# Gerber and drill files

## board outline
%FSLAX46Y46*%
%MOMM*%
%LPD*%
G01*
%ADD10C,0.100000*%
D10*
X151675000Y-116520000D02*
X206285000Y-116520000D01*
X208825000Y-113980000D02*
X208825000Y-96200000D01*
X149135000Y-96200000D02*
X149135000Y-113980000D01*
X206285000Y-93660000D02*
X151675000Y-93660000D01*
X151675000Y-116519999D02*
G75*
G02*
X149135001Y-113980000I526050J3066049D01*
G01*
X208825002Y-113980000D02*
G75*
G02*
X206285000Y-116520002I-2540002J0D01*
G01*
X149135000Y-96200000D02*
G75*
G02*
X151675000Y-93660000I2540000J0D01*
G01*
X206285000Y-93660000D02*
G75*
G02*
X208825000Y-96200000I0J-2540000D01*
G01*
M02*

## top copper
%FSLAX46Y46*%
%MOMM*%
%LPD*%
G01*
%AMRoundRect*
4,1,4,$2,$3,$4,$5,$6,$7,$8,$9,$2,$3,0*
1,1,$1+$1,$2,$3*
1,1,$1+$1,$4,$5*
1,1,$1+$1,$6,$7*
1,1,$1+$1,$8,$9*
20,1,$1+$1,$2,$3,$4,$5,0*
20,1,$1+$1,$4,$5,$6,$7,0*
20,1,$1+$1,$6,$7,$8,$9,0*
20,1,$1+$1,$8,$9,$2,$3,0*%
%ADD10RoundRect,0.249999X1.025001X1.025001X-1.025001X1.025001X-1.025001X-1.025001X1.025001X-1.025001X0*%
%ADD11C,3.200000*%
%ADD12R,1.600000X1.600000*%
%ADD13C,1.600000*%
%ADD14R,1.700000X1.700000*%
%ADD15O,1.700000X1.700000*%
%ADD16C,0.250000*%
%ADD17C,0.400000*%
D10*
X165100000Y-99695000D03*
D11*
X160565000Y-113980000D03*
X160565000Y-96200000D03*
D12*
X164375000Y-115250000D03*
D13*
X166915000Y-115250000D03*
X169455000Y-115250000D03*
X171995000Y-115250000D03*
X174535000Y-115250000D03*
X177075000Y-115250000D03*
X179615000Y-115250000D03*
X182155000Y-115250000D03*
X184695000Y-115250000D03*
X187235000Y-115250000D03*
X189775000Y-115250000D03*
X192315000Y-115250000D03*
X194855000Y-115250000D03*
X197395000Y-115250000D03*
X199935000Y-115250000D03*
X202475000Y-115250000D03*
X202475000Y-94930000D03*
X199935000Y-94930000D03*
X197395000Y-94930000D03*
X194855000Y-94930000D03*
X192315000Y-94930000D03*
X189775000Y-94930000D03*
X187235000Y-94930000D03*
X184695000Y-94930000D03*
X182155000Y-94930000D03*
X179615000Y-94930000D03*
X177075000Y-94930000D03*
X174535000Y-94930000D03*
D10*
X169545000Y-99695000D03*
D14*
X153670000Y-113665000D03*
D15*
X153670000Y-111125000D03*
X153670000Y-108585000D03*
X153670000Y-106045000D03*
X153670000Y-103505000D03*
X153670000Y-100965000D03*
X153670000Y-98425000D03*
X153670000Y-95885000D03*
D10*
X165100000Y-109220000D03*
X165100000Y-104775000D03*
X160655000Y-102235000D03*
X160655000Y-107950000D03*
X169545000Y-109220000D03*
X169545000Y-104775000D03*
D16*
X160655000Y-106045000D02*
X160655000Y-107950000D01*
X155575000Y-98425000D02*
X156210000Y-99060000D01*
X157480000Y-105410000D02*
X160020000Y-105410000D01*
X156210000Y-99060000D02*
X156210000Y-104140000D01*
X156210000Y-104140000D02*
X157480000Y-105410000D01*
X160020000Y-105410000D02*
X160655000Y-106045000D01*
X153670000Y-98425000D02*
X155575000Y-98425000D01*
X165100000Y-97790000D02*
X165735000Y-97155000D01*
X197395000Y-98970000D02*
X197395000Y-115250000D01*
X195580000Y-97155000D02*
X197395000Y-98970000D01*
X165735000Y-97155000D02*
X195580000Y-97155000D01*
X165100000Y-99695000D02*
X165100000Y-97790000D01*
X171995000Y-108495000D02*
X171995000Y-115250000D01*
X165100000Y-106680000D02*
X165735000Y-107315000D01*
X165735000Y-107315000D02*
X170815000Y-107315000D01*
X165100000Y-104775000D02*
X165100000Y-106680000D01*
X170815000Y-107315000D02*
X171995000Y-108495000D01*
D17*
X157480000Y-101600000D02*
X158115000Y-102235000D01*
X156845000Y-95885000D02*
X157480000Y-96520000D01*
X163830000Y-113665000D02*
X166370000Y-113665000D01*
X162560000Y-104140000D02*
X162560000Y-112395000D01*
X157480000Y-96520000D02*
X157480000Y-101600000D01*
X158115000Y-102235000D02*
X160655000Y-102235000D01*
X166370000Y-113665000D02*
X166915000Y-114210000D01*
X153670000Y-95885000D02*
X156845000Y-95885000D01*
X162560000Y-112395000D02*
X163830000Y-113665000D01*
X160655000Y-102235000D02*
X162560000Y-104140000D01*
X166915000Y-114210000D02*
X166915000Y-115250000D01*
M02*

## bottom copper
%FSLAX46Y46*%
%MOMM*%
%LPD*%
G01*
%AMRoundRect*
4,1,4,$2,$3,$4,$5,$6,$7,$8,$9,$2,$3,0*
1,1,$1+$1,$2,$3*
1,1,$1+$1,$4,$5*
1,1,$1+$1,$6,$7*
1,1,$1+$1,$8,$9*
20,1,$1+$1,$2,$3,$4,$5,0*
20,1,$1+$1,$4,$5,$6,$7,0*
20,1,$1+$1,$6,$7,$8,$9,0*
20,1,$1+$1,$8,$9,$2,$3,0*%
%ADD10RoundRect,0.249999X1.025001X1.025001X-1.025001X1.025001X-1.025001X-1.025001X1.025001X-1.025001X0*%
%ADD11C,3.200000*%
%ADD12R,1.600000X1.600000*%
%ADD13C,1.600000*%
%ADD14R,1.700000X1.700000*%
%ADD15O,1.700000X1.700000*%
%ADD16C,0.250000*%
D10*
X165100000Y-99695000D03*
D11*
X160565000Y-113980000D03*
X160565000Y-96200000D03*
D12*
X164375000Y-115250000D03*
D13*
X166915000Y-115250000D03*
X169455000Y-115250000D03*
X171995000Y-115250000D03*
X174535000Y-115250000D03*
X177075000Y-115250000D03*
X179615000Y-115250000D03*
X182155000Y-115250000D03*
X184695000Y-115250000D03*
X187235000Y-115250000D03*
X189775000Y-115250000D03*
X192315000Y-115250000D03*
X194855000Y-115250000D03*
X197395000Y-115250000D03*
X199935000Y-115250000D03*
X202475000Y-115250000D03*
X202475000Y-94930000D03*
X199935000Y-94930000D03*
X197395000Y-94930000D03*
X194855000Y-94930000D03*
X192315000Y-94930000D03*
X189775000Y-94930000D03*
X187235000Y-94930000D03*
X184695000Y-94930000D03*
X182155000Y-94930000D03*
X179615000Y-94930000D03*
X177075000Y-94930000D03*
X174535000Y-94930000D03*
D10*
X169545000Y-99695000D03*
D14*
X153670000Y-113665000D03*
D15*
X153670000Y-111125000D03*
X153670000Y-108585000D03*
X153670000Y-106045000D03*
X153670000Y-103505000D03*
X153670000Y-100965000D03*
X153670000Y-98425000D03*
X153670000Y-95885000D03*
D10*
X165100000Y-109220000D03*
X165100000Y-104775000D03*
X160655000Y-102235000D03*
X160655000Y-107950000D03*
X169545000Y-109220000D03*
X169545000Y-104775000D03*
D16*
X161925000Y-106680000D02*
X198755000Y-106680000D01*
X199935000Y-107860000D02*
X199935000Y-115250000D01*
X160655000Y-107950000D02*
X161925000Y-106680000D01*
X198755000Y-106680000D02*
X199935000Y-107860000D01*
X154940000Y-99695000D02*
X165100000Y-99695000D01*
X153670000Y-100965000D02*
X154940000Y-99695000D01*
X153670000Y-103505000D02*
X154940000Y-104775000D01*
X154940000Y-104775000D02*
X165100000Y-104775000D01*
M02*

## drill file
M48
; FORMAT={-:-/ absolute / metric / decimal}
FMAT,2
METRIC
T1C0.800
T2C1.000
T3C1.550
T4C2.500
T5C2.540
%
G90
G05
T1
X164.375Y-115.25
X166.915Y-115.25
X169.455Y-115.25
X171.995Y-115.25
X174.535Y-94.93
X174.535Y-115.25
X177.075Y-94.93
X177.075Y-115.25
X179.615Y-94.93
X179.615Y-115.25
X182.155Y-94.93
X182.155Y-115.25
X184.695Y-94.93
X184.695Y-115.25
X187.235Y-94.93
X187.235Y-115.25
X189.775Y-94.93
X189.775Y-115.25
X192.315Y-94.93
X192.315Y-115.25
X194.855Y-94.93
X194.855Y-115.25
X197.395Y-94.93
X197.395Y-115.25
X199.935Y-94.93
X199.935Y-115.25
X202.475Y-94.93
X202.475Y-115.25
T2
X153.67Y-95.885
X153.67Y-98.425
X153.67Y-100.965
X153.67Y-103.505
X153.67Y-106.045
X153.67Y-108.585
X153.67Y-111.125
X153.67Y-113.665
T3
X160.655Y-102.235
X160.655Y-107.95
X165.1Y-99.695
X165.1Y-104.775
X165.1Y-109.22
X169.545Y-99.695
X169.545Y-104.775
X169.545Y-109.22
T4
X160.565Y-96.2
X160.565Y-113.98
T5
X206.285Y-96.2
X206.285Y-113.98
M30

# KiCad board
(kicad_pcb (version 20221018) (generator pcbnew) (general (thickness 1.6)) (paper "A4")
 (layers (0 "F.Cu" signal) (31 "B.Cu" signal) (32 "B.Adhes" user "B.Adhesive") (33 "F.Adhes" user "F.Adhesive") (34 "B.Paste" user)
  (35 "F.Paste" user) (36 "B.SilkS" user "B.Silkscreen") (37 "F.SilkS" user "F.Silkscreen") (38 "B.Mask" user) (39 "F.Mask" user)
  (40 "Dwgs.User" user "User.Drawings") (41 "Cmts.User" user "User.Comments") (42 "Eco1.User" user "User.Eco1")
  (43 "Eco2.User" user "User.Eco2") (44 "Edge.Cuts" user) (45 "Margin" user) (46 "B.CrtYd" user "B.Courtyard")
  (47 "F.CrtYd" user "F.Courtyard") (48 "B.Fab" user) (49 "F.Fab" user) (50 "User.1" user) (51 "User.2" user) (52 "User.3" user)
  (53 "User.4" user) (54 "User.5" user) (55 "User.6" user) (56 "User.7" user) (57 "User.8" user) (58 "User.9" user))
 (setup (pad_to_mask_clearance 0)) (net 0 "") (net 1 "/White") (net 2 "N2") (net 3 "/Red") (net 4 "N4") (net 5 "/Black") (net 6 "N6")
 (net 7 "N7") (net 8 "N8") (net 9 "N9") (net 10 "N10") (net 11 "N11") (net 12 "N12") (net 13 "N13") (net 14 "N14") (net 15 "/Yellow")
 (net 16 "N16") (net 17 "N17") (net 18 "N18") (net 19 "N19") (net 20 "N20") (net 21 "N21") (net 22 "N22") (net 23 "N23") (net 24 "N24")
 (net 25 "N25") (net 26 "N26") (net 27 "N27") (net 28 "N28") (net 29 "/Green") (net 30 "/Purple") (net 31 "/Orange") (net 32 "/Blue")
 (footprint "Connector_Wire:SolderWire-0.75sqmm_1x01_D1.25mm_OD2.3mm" (layer "F.Cu") (at 165.1 99.695 180)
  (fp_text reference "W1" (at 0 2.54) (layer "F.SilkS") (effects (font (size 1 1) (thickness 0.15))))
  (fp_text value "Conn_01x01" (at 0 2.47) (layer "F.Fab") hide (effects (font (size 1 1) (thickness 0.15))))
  (pad "1" thru_hole roundrect (at 0 0 180) (size 2.55 2.55) (drill 1.55) (layers "*.Cu" "*.Mask") (roundrect_rratio 0.098039)
   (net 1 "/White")))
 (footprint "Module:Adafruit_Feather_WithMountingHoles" (layer "F.Cu") (at 164.375 115.25 90)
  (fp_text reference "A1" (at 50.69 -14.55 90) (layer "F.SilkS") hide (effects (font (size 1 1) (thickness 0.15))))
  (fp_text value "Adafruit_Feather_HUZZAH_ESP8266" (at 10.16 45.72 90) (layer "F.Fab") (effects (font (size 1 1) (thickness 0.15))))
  (fp_line (start -1.27 -12.7) (end -1.27 41.91) (stroke (width 0.1) (type solid)) (layer "Edge.Cuts"))
  (fp_line (start 1.27 44.45) (end 19.05 44.45) (stroke (width 0.1) (type solid)) (layer "Edge.Cuts"))
  (fp_line (start 19.05 -15.24) (end 1.27 -15.24) (stroke (width 0.1) (type solid)) (layer "Edge.Cuts"))
  (fp_line (start 21.59 41.91) (end 21.59 -12.7) (stroke (width 0.1) (type solid)) (layer "Edge.Cuts"))
  (fp_arc (start -1.269999 -12.7) (mid -0.403653 -14.373653) (end 1.27 -15.239999) (stroke (width 0.1) (type solid)) (layer "Edge.Cuts"))
  (fp_arc (start 1.27 44.450002) (mid -0.526052 43.706052) (end -1.27 41.91) (stroke (width 0.1) (type solid)) (layer "Edge.Cuts"))
  (fp_arc (start 19.05 -15.24) (mid 20.846051 -14.496051) (end 21.59 -12.7) (stroke (width 0.1) (type solid)) (layer "Edge.Cuts"))
  (fp_arc (start 21.59 41.91) (mid 20.846051 43.706051) (end 19.05 44.45) (stroke (width 0.1) (type solid)) (layer "Edge.Cuts"))
  (pad "" np_thru_hole circle (at 1.27 -3.81) (size 3.2 3.2) (drill 2.5) (layers "*.Cu" "*.Mask"))
  (pad "" np_thru_hole circle (at 1.27 41.91) (size 2.54 2.54) (drill 2.54) (layers "*.Cu" "*.Mask"))
  (pad "" np_thru_hole circle (at 19.05 -3.81) (size 3.2 3.2) (drill 2.5) (layers "*.Cu" "*.Mask"))
  (pad "" np_thru_hole circle (at 19.05 41.91) (size 2.54 2.54) (drill 2.54) (layers "*.Cu" "*.Mask"))
  (pad "1" thru_hole rect (at 0 0 270) (size 1.6 1.6) (drill 0.8) (layers "*.Cu" "*.Mask") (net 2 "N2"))
  (pad "2" thru_hole circle (at 0 2.54 270) (size 1.6 1.6) (drill 0.8) (layers "*.Cu" "*.Mask") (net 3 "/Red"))
  (pad "3" thru_hole circle (at 0 5.08 270) (size 1.6 1.6) (drill 0.8) (layers "*.Cu" "*.Mask") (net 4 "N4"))
  (pad "4" thru_hole circle (at 0 7.62 270) (size 1.6 1.6) (drill 0.8) (layers "*.Cu" "*.Mask") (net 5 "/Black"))
  (pad "5" thru_hole circle (at 0 10.16 270) (size 1.6 1.6) (drill 0.8) (layers "*.Cu" "*.Mask") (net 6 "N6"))
  (pad "6" thru_hole circle (at 0 12.7 270) (size 1.6 1.6) (drill 0.8) (layers "*.Cu" "*.Mask") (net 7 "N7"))
  (pad "7" thru_hole circle (at 0 15.24 270) (size 1.6 1.6) (drill 0.8) (layers "*.Cu" "*.Mask") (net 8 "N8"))
  (pad "8" thru_hole circle (at 0 17.78 270) (size 1.6 1.6) (drill 0.8) (layers "*.Cu" "*.Mask") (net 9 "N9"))
  (pad "9" thru_hole circle (at 0 20.32 270) (size 1.6 1.6) (drill 0.8) (layers "*.Cu" "*.Mask") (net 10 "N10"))
  (pad "10" thru_hole circle (at 0 22.86 270) (size 1.6 1.6) (drill 0.8) (layers "*.Cu" "*.Mask") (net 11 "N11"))
  (pad "11" thru_hole circle (at 0 25.4 270) (size 1.6 1.6) (drill 0.8) (layers "*.Cu" "*.Mask") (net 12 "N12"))
  (pad "12" thru_hole circle (at 0 27.94 270) (size 1.6 1.6) (drill 0.8) (layers "*.Cu" "*.Mask") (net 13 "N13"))
  (pad "13" thru_hole circle (at 0 30.48 270) (size 1.6 1.6) (drill 0.8) (layers "*.Cu" "*.Mask") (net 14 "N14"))
  (pad "14" thru_hole circle (at 0 33.02 270) (size 1.6 1.6) (drill 0.8) (layers "*.Cu" "*.Mask") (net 1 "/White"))
  (pad "15" thru_hole circle (at 0 35.56 270) (size 1.6 1.6) (drill 0.8) (layers "*.Cu" "*.Mask") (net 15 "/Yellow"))
  (pad "16" thru_hole circle (at 0 38.1 270) (size 1.6 1.6) (drill 0.8) (layers "*.Cu" "*.Mask") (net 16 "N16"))
  (pad "17" thru_hole circle (at 20.32 38.1 270) (size 1.6 1.6) (drill 0.8) (layers "*.Cu" "*.Mask") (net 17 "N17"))
  (pad "18" thru_hole circle (at 20.32 35.56 270) (size 1.6 1.6) (drill 0.8) (layers "*.Cu" "*.Mask") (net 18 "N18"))
  (pad "19" thru_hole circle (at 20.32 33.02 270) (size 1.6 1.6) (drill 0.8) (layers "*.Cu" "*.Mask") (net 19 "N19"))
  (pad "20" thru_hole circle (at 20.32 30.48 270) (size 1.6 1.6) (drill 0.8) (layers "*.Cu" "*.Mask") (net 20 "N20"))
  (pad "21" thru_hole circle (at 20.32 27.94 270) (size 1.6 1.6) (drill 0.8) (layers "*.Cu" "*.Mask") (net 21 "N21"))
  (pad "22" thru_hole circle (at 20.32 25.4 270) (size 1.6 1.6) (drill 0.8) (layers "*.Cu" "*.Mask") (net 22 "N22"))
  (pad "23" thru_hole circle (at 20.32 22.86 270) (size 1.6 1.6) (drill 0.8) (layers "*.Cu" "*.Mask") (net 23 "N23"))
  (pad "24" thru_hole circle (at 20.32 20.32 270) (size 1.6 1.6) (drill 0.8) (layers "*.Cu" "*.Mask") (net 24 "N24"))
  (pad "25" thru_hole circle (at 20.32 17.78 270) (size 1.6 1.6) (drill 0.8) (layers "*.Cu" "*.Mask") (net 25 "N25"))
  (pad "26" thru_hole circle (at 20.32 15.24 270) (size 1.6 1.6) (drill 0.8) (layers "*.Cu" "*.Mask") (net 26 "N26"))
  (pad "27" thru_hole circle (at 20.32 12.7 270) (size 1.6 1.6) (drill 0.8) (layers "*.Cu" "*.Mask") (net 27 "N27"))
  (pad "28" thru_hole circle (at 20.32 10.16 270) (size 1.6 1.6) (drill 0.8) (layers "*.Cu" "*.Mask") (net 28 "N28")))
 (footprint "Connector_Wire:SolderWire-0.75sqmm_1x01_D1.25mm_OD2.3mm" (layer "F.Cu") (at 169.545 99.695 180)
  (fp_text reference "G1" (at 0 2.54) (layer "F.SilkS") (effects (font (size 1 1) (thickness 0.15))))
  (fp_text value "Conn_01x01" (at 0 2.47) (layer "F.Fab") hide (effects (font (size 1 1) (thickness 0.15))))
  (pad "1" thru_hole roundrect (at 0 0 180) (size 2.55 2.55) (drill 1.55) (layers "*.Cu" "*.Mask") (roundrect_rratio 0.098039)
   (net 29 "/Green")))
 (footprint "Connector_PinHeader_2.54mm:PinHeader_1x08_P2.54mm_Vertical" (layer "F.Cu") (at 153.67 113.665 180)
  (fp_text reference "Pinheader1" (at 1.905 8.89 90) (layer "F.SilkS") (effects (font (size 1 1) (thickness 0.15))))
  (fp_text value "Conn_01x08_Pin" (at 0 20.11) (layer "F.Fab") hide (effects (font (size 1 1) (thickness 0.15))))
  (pad "1" thru_hole rect (at 0 0 180) (size 1.7 1.7) (drill 1) (layers "*.Cu" "*.Mask") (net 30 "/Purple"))
  (pad "2" thru_hole oval (at 0 2.54 180) (size 1.7 1.7) (drill 1) (layers "*.Cu" "*.Mask") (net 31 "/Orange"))
  (pad "3" thru_hole oval (at 0 5.08 180) (size 1.7 1.7) (drill 1) (layers "*.Cu" "*.Mask") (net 29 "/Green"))
  (pad "4" thru_hole oval (at 0 7.62 180) (size 1.7 1.7) (drill 1) (layers "*.Cu" "*.Mask") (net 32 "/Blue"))
  (pad "5" thru_hole oval (at 0 10.16 180) (size 1.7 1.7) (drill 1) (layers "*.Cu" "*.Mask") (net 5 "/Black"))
  (pad "6" thru_hole oval (at 0 12.7 180) (size 1.7 1.7) (drill 1) (layers "*.Cu" "*.Mask") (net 1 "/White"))
  (pad "7" thru_hole oval (at 0 15.24 180) (size 1.7 1.7) (drill 1) (layers "*.Cu" "*.Mask") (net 15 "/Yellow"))
  (pad "8" thru_hole oval (at 0 17.78 180) (size 1.7 1.7) (drill 1) (layers "*.Cu" "*.Mask") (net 3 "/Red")))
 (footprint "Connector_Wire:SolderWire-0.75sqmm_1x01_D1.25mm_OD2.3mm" (layer "F.Cu") (at 165.1 109.22 180)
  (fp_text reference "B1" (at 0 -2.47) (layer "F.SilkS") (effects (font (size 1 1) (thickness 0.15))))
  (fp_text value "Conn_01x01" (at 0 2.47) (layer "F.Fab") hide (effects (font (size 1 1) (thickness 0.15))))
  (pad "1" thru_hole roundrect (at 0 0 180) (size 2.55 2.55) (drill 1.55) (layers "*.Cu" "*.Mask") (roundrect_rratio 0.098039)
   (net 32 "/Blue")))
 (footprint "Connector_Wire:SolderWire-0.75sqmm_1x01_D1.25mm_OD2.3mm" (layer "F.Cu") (at 165.1 104.775 180)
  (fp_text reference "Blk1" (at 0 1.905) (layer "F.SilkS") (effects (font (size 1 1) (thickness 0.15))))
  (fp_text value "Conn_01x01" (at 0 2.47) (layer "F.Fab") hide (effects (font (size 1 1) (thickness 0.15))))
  (pad "1" thru_hole roundrect (at 0 0 180) (size 2.55 2.55) (drill 1.55) (layers "*.Cu" "*.Mask") (roundrect_rratio 0.098039)
   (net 5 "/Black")))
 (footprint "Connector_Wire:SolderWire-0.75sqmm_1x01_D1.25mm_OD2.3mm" (layer "F.Cu") (at 160.655 102.235 180)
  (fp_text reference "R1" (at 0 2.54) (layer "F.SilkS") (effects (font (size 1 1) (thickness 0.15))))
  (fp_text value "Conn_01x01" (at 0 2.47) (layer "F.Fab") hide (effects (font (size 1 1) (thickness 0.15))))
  (pad "1" thru_hole roundrect (at 0 0 180) (size 2.55 2.55) (drill 1.55) (layers "*.Cu" "*.Mask") (roundrect_rratio 0.098039)
   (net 3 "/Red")))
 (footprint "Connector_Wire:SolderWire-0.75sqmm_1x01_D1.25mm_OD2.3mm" (layer "F.Cu") (at 160.655 107.95 180)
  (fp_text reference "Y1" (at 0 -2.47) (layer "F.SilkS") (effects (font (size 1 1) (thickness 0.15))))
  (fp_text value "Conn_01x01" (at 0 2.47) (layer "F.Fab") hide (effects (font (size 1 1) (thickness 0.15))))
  (pad "1" thru_hole roundrect (at 0 0 180) (size 2.55 2.55) (drill 1.55) (layers "*.Cu" "*.Mask") (roundrect_rratio 0.098039)
   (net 15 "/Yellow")))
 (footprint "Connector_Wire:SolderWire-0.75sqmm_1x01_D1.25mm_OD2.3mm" (layer "F.Cu") (at 169.545 109.22 180)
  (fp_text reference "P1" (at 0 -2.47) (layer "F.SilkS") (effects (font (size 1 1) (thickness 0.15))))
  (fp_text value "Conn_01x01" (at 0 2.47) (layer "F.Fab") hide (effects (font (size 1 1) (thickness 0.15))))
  (pad "1" thru_hole roundrect (at 0 0 180) (size 2.55 2.55) (drill 1.55) (layers "*.Cu" "*.Mask") (roundrect_rratio 0.098039)
   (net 30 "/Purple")))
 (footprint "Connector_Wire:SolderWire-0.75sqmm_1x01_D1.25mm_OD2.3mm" (layer "F.Cu") (at 169.545 104.775 180)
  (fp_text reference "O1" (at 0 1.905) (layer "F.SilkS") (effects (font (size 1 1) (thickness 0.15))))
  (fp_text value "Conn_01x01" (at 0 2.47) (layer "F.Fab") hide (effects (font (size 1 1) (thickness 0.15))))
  (pad "1" thru_hole roundrect (at 0 0 180) (size 2.55 2.55) (drill 1.55) (layers "*.Cu" "*.Mask") (roundrect_rratio 0.098039)
   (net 31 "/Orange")))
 (segment (start 160.655 106.045) (end 160.655 107.95) (width 0.25) (layer "F.Cu") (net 15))
 (segment (start 155.575 98.425) (end 156.21 99.06) (width 0.25) (layer "F.Cu") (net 15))
 (segment (start 157.48 105.41) (end 160.02 105.41) (width 0.25) (layer "F.Cu") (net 15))
 (segment (start 156.21 99.06) (end 156.21 104.14) (width 0.25) (layer "F.Cu") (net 15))
 (segment (start 156.21 104.14) (end 157.48 105.41) (width 0.25) (layer "F.Cu") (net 15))
 (segment (start 160.02 105.41) (end 160.655 106.045) (width 0.25) (layer "F.Cu") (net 15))
 (segment (start 153.67 98.425) (end 155.575 98.425) (width 0.25) (layer "F.Cu") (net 15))
 (segment (start 161.925 106.68) (end 198.755 106.68) (width 0.25) (layer "B.Cu") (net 15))
 (segment (start 199.935 107.86) (end 199.935 115.25) (width 0.25) (layer "B.Cu") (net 15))
 (segment (start 160.655 107.95) (end 161.925 106.68) (width 0.25) (layer "B.Cu") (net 15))
 (segment (start 198.755 106.68) (end 199.935 107.86) (width 0.25) (layer "B.Cu") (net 15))
 (segment (start 165.1 97.79) (end 165.735 97.155) (width 0.25) (layer "F.Cu") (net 1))
 (segment (start 197.395 98.97) (end 197.395 115.25) (width 0.25) (layer "F.Cu") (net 1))
 (segment (start 195.58 97.155) (end 197.395 98.97) (width 0.25) (layer "F.Cu") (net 1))
 (segment (start 165.735 97.155) (end 195.58 97.155) (width 0.25) (layer "F.Cu") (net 1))
 (segment (start 165.1 99.695) (end 165.1 97.79) (width 0.25) (layer "F.Cu") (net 1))
 (segment (start 154.94 99.695) (end 165.1 99.695) (width 0.25) (layer "B.Cu") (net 1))
 (segment (start 153.67 100.965) (end 154.94 99.695) (width 0.25) (layer "B.Cu") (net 1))
 (segment (start 171.995 108.495) (end 171.995 115.25) (width 0.25) (layer "F.Cu") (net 5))
 (segment (start 165.1 106.68) (end 165.735 107.315) (width 0.25) (layer "F.Cu") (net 5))
 (segment (start 165.735 107.315) (end 170.815 107.315) (width 0.25) (layer "F.Cu") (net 5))
 (segment (start 165.1 104.775) (end 165.1 106.68) (width 0.25) (layer "F.Cu") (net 5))
 (segment (start 170.815 107.315) (end 171.995 108.495) (width 0.25) (layer "F.Cu") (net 5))
 (segment (start 153.67 103.505) (end 154.94 104.775) (width 0.25) (layer "B.Cu") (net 5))
 (segment (start 154.94 104.775) (end 165.1 104.775) (width 0.25) (layer "B.Cu") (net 5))
 (segment (start 157.48 101.6) (end 158.115 102.235) (width 0.4) (layer "F.Cu") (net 3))
 (segment (start 156.845 95.885) (end 157.48 96.52) (width 0.4) (layer "F.Cu") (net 3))
 (segment (start 163.83 113.665) (end 166.37 113.665) (width 0.4) (layer "F.Cu") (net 3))
 (segment (start 162.56 104.14) (end 162.56 112.395) (width 0.4) (layer "F.Cu") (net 3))
 (segment (start 157.48 96.52) (end 157.48 101.6) (width 0.4) (layer "F.Cu") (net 3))
 (segment (start 158.115 102.235) (end 160.655 102.235) (width 0.4) (layer "F.Cu") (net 3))
 (segment (start 166.37 113.665) (end 166.915 114.21) (width 0.4) (layer "F.Cu") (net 3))
 (segment (start 153.67 95.885) (end 156.845 95.885) (width 0.4) (layer "F.Cu") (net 3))
 (segment (start 162.56 112.395) (end 163.83 113.665) (width 0.4) (layer "F.Cu") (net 3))
 (segment (start 160.655 102.235) (end 162.56 104.14) (width 0.4) (layer "F.Cu") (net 3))
 (segment (start 166.915 114.21) (end 166.915 115.25) (width 0.4) (layer "F.Cu") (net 3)))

